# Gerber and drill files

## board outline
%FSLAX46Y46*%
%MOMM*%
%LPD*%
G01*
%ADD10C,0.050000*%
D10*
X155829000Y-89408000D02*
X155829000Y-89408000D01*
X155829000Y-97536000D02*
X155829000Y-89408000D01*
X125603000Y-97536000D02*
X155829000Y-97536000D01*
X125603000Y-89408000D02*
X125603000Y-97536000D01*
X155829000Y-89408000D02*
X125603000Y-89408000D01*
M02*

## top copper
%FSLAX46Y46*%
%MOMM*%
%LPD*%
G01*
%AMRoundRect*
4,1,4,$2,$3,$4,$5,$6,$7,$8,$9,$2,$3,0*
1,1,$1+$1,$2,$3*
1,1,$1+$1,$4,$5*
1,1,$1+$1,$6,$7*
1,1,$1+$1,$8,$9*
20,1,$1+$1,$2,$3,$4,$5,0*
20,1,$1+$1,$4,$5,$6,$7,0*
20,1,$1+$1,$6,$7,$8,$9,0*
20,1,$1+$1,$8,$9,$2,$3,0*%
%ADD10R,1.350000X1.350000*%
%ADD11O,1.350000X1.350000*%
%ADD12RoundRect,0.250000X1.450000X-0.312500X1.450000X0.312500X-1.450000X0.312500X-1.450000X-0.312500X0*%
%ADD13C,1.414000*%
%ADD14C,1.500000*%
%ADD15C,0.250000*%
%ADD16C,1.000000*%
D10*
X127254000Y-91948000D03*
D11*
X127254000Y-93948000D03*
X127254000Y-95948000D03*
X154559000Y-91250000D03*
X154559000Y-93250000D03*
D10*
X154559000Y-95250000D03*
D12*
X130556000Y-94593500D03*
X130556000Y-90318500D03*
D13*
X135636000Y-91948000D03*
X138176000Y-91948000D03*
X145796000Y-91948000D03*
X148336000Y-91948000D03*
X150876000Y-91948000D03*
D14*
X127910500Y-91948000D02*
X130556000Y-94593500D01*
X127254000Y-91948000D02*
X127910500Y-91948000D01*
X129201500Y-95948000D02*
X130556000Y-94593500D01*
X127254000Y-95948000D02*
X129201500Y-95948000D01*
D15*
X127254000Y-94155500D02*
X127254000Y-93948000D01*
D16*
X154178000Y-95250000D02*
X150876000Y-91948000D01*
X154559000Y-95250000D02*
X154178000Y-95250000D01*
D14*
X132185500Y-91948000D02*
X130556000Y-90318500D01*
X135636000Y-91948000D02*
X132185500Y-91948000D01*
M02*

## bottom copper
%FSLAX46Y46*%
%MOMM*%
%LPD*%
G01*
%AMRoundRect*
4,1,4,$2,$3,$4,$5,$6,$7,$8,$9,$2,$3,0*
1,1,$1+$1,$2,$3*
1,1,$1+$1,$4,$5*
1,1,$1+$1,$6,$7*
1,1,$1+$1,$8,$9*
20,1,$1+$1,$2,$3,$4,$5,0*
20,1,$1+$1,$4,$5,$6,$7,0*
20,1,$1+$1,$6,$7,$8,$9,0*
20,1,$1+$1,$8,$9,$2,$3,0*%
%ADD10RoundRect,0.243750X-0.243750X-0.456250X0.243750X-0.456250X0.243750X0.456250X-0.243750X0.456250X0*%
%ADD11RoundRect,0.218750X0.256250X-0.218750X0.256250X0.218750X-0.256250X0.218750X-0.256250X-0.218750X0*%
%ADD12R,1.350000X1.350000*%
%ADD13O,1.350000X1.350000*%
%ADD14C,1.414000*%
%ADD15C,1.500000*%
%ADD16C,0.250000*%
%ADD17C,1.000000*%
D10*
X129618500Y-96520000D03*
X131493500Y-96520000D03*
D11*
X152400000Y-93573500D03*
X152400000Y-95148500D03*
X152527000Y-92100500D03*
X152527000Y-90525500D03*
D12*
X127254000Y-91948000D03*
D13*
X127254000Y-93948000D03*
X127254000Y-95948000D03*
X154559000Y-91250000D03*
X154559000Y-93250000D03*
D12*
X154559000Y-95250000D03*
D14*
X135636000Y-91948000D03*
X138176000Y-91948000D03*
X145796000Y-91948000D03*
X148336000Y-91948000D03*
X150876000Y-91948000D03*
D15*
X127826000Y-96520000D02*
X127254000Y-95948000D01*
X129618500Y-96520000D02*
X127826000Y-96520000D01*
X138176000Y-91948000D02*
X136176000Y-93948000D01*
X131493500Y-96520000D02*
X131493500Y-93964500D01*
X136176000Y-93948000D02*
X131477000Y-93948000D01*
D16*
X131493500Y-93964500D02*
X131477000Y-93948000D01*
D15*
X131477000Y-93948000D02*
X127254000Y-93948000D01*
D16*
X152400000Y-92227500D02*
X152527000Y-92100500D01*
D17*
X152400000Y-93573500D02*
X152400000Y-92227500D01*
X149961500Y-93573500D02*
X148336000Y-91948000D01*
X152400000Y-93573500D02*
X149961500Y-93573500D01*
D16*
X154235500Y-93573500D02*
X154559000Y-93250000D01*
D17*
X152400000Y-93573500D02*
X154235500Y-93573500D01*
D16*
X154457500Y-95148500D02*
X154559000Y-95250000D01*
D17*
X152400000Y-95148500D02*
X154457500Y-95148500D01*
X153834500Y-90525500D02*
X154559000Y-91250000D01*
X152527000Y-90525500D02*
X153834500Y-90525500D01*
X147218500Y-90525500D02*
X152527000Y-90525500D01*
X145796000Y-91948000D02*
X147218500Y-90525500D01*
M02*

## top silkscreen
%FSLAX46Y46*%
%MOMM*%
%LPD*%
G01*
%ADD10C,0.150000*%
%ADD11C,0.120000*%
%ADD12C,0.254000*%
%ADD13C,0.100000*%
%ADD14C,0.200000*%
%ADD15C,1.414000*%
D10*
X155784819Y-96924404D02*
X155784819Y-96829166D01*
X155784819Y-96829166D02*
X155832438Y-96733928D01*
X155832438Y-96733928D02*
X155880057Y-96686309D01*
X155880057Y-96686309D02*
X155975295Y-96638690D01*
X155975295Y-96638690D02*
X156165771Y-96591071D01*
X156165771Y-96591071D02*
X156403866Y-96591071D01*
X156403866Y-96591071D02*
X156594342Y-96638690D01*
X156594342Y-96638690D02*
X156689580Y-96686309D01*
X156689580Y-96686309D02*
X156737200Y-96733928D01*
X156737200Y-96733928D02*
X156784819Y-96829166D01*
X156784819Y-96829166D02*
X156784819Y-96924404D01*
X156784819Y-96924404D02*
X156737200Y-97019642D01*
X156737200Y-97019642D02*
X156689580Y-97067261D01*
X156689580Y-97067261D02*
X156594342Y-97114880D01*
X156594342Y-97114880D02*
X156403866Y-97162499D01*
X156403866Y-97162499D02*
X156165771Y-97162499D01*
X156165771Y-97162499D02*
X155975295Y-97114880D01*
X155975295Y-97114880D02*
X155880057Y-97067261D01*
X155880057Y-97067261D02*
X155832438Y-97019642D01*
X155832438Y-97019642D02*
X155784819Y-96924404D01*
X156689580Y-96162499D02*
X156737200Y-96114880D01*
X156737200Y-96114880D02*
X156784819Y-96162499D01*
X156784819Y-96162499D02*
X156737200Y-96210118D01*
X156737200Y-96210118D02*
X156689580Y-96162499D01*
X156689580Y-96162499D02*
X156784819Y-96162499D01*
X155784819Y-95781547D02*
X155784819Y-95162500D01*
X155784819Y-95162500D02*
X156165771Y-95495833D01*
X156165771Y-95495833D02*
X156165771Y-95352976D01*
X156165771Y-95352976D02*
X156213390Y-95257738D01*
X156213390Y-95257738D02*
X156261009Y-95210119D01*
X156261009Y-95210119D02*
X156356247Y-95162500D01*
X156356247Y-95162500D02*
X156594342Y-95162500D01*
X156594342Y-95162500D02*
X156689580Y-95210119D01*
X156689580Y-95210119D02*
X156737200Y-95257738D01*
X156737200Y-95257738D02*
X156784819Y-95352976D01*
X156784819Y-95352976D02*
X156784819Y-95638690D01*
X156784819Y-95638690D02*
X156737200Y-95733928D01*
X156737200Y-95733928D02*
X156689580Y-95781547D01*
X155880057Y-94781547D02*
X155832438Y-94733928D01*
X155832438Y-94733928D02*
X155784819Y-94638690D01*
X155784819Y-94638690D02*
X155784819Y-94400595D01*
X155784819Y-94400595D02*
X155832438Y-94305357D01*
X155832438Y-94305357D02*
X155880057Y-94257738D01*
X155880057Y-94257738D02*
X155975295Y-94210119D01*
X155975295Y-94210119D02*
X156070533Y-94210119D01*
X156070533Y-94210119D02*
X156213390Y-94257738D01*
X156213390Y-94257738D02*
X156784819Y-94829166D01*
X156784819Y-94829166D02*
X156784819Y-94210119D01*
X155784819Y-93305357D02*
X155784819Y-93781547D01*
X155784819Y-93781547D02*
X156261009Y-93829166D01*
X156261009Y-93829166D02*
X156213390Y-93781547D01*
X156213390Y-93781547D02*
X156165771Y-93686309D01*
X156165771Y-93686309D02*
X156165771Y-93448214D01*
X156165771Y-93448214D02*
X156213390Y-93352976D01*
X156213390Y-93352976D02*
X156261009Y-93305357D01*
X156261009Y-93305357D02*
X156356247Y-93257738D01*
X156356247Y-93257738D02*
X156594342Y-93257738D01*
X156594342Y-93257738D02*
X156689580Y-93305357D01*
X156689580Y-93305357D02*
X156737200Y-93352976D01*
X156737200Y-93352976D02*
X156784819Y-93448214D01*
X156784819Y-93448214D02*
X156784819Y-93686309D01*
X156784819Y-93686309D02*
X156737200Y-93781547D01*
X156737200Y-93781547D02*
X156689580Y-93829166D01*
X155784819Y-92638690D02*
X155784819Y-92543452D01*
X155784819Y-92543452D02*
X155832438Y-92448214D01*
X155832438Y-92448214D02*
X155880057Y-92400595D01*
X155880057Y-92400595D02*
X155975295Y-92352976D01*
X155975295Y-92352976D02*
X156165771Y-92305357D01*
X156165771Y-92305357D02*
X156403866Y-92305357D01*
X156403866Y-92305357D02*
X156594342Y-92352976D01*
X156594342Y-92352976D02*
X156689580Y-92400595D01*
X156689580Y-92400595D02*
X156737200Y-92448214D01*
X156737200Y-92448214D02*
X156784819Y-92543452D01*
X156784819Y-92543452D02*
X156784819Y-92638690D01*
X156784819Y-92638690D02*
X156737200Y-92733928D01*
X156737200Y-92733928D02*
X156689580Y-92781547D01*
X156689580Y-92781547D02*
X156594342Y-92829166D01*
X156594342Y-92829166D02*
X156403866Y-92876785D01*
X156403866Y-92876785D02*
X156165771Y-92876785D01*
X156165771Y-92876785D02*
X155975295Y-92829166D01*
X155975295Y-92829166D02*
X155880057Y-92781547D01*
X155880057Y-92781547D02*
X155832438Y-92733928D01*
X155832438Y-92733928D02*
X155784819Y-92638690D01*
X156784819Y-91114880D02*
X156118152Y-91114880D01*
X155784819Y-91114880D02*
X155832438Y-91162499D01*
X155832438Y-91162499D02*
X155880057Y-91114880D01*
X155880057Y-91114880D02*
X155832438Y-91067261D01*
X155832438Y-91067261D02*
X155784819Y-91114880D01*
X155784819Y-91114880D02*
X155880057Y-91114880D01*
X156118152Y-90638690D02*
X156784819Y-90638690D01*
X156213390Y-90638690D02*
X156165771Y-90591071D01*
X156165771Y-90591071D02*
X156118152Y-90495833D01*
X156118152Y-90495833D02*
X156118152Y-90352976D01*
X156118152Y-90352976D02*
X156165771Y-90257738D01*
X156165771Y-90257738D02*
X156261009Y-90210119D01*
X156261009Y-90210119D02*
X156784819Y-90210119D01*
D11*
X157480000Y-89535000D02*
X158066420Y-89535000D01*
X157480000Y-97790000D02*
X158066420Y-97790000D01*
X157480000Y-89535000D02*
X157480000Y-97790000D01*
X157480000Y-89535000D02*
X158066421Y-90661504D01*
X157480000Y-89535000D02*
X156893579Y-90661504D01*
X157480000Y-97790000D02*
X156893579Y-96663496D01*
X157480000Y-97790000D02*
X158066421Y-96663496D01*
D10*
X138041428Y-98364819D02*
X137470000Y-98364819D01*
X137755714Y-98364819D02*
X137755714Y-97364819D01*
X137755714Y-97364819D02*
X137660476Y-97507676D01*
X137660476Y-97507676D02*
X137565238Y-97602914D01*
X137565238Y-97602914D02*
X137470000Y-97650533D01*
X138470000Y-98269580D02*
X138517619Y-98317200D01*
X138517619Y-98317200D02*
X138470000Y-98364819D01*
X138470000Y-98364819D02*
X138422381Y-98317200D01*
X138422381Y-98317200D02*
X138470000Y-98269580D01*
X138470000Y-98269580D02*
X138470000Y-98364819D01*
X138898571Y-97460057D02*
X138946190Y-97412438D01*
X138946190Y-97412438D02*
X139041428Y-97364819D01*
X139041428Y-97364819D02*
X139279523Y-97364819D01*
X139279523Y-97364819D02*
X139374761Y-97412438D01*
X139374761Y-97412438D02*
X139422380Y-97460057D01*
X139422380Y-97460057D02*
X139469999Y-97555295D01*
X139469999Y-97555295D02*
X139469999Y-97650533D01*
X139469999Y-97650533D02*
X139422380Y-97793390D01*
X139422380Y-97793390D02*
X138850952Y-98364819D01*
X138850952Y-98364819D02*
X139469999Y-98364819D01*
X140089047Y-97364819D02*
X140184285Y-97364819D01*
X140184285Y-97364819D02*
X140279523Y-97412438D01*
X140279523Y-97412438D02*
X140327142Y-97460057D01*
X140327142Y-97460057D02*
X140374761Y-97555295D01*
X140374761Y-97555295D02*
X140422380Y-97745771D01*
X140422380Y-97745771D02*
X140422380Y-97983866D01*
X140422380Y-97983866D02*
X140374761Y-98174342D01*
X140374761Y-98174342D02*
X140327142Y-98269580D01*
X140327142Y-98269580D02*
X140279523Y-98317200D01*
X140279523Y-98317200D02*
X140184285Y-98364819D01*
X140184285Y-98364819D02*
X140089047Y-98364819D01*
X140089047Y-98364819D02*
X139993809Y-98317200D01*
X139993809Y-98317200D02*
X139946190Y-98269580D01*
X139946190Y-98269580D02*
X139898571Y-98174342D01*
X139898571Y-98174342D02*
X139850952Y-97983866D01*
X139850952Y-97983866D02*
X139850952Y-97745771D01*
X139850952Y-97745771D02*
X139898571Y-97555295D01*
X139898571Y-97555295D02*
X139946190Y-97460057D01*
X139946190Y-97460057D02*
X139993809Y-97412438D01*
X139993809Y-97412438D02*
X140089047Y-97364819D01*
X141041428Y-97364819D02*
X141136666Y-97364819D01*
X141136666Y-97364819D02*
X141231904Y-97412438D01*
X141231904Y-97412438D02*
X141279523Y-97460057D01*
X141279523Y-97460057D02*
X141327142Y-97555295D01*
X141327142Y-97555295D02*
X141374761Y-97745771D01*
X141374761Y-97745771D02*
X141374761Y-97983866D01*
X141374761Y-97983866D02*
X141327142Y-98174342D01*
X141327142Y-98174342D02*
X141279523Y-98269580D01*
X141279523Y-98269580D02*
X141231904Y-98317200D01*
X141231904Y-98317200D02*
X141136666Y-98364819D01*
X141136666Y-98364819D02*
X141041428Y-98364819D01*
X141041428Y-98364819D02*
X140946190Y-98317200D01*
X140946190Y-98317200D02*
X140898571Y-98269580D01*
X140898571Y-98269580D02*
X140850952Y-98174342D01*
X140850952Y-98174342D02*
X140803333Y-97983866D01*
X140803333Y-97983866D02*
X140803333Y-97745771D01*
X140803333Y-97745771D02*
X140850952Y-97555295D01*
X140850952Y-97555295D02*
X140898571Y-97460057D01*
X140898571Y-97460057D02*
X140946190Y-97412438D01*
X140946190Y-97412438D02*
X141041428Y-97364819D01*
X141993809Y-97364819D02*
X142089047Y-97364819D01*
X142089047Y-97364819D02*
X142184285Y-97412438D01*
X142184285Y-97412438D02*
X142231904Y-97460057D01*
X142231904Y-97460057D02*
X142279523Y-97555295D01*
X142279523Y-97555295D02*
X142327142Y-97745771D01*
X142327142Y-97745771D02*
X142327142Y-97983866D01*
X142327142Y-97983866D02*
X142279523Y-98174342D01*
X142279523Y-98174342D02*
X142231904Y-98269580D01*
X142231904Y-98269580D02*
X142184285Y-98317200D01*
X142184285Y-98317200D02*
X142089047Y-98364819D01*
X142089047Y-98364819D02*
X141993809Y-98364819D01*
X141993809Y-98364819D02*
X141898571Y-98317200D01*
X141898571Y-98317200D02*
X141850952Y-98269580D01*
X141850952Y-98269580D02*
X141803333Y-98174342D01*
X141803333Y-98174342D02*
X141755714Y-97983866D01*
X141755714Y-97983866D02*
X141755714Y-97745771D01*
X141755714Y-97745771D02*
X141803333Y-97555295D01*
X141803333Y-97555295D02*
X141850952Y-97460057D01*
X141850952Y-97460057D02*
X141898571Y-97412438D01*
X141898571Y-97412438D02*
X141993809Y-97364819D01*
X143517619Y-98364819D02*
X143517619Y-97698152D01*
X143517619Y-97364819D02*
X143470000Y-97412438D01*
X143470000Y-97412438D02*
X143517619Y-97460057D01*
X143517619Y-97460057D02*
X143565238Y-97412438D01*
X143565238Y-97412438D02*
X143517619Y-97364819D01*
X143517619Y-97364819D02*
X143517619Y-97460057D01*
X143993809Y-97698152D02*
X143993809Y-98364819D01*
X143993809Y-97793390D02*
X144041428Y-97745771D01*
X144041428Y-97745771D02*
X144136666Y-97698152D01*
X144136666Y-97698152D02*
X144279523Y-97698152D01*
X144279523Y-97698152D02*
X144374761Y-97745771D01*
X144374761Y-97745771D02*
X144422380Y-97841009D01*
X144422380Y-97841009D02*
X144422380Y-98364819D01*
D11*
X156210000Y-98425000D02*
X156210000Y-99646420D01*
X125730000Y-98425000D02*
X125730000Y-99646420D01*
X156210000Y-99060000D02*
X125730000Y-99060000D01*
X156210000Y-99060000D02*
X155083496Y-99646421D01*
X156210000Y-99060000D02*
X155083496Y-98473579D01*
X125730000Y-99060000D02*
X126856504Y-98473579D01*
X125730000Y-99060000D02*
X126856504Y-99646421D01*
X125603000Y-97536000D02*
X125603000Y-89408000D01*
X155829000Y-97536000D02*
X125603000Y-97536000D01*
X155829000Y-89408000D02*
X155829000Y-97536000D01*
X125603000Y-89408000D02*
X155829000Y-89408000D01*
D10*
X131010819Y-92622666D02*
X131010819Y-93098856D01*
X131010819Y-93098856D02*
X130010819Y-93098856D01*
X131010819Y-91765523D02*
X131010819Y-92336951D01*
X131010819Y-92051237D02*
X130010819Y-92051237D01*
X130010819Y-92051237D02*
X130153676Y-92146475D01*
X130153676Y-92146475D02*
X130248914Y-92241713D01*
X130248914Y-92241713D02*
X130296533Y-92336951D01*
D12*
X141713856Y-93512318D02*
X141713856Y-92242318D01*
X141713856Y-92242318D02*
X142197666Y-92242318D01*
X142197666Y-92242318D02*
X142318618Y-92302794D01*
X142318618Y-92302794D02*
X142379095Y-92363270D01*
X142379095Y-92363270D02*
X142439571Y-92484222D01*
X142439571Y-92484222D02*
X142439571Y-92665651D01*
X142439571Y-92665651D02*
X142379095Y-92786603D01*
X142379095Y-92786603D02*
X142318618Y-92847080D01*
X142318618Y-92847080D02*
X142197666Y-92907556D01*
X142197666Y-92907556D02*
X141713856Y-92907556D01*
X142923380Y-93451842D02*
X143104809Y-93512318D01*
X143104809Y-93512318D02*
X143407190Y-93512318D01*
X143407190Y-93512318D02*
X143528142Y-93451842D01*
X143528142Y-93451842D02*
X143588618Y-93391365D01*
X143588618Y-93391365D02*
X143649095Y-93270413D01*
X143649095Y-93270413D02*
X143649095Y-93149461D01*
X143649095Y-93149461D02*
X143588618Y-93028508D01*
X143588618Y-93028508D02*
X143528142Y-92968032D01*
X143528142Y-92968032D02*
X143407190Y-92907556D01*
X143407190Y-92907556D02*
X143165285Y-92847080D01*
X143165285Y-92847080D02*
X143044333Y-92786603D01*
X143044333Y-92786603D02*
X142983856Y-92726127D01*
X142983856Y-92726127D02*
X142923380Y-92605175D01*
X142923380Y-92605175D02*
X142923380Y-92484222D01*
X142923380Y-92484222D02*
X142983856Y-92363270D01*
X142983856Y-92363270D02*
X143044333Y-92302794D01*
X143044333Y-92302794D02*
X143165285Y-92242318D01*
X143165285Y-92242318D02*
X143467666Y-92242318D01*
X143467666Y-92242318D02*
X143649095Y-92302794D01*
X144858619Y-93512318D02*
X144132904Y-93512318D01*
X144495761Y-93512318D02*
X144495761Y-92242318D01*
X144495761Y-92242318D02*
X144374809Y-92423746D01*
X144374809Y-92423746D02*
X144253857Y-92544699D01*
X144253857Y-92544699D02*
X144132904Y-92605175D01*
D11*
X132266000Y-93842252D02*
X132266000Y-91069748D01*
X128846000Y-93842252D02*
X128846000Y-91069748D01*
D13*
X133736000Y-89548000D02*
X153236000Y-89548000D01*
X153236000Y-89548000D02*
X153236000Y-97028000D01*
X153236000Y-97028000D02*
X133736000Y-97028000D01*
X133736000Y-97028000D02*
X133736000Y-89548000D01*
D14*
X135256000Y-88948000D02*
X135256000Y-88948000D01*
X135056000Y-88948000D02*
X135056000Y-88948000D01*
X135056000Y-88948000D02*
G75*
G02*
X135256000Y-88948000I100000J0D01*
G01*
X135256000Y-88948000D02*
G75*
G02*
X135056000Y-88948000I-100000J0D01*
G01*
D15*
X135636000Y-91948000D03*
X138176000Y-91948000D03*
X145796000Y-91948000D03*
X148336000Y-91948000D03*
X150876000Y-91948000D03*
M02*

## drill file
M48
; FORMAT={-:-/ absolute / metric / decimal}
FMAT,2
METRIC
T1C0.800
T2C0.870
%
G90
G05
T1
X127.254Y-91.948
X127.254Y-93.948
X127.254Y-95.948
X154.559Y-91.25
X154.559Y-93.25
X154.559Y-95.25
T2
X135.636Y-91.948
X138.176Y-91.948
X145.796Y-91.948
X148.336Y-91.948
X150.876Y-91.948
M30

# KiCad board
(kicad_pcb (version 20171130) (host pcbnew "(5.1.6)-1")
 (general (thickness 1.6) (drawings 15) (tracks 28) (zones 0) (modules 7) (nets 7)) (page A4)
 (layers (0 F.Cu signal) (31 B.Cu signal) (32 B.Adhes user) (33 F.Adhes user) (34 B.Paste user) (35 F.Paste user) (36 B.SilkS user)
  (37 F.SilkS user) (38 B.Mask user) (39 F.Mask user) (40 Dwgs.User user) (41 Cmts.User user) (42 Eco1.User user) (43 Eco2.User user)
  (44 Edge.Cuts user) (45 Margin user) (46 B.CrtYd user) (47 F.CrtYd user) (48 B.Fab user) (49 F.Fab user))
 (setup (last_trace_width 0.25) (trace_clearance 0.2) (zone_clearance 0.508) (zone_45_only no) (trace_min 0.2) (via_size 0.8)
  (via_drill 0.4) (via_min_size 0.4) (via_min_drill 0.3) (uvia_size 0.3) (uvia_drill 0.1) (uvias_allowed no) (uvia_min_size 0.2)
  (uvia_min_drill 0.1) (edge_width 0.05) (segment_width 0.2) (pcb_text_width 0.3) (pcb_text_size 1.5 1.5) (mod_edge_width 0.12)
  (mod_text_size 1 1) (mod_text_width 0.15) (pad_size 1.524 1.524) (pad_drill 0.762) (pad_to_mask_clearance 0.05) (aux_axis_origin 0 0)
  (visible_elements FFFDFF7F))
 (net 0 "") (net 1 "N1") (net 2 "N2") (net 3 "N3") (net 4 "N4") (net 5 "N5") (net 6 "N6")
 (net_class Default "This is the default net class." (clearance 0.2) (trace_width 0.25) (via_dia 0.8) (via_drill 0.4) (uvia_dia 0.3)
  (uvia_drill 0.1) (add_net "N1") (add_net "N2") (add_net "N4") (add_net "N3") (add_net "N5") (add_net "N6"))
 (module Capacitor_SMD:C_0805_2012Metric (layer B.Cu) (at 130.556 96.52)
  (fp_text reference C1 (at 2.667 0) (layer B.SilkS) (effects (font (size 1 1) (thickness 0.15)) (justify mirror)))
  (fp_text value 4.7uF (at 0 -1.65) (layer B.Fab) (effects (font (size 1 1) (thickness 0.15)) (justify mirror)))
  (pad 1 smd roundrect (at -0.9375 0) (size 0.975 1.4) (layers B.Cu B.Paste B.Mask) (roundrect_rratio 0.25) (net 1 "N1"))
  (pad 2 smd roundrect (at 0.9375 0) (size 0.975 1.4) (layers B.Cu B.Paste B.Mask) (roundrect_rratio 0.25) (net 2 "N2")))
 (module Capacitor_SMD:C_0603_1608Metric (layer B.Cu) (at 152.4 94.361 90)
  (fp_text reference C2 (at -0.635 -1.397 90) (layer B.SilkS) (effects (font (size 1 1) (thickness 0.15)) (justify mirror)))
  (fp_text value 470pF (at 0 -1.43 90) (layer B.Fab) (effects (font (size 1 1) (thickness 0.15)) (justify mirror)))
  (pad 2 smd roundrect (at 0.7875 0 90) (size 0.875 0.95) (layers B.Cu B.Paste B.Mask) (roundrect_rratio 0.25) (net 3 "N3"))
  (pad 1 smd roundrect (at -0.7875 0 90) (size 0.875 0.95) (layers B.Cu B.Paste B.Mask) (roundrect_rratio 0.25) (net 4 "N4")))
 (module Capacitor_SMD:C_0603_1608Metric (layer B.Cu) (at 152.527 91.313 90)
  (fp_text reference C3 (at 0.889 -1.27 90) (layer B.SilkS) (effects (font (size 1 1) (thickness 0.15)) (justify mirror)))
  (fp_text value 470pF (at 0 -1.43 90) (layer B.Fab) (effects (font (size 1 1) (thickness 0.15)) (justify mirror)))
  (pad 1 smd roundrect (at -0.7875 0 90) (size 0.875 0.95) (layers B.Cu B.Paste B.Mask) (roundrect_rratio 0.25) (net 3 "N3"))
  (pad 2 smd roundrect (at 0.7875 0 90) (size 0.875 0.95) (layers B.Cu B.Paste B.Mask) (roundrect_rratio 0.25) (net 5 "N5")))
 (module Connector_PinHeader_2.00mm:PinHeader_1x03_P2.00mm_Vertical (layer B.Cu) (at 127.254 91.948 180)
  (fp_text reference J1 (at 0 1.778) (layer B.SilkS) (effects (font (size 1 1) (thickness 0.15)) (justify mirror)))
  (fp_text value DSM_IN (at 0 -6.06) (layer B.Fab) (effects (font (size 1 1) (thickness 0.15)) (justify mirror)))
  (pad 1 thru_hole rect (at 0 0 180) (size 1.35 1.35) (drill 0.8) (layers *.Cu *.Mask) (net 1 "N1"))
  (pad 2 thru_hole oval (at 0 -2 180) (size 1.35 1.35) (drill 0.8) (layers *.Cu *.Mask) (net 2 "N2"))
  (pad 3 thru_hole oval (at 0 -4 180) (size 1.35 1.35) (drill 0.8) (layers *.Cu *.Mask) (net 1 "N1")))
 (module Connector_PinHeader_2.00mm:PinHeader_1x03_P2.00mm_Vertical (layer B.Cu) (at 154.559 95.25)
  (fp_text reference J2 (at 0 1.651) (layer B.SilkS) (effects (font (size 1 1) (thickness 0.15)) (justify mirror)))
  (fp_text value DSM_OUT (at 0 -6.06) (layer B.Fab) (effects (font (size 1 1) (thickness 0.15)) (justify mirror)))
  (pad 3 thru_hole oval (at 0 -4) (size 1.35 1.35) (drill 0.8) (layers *.Cu *.Mask) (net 5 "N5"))
  (pad 2 thru_hole oval (at 0 -2) (size 1.35 1.35) (drill 0.8) (layers *.Cu *.Mask) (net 3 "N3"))
  (pad 1 thru_hole rect (at 0 0) (size 1.35 1.35) (drill 0.8) (layers *.Cu *.Mask) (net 4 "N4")))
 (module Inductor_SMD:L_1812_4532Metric (layer F.Cu) (at 130.556 92.456 90)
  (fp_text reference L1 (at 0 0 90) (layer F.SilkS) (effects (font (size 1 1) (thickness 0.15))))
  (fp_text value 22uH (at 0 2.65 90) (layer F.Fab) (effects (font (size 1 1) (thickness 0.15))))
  (fp_line (start -1.386252 1.71) (end 1.386252 1.71) (layer F.SilkS) (width 0.12))
  (fp_line (start -1.386252 -1.71) (end 1.386252 -1.71) (layer F.SilkS) (width 0.12))
  (pad 1 smd roundrect (at -2.1375 0 90) (size 1.125 3.4) (layers F.Cu F.Paste F.Mask) (roundrect_rratio 0.222222) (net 1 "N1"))
  (pad 2 smd roundrect (at 2.1375 0 90) (size 1.125 3.4) (layers F.Cu F.Paste F.Mask) (roundrect_rratio 0.222222) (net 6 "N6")))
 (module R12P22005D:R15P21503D (layer F.Cu) (at 135.636 91.948)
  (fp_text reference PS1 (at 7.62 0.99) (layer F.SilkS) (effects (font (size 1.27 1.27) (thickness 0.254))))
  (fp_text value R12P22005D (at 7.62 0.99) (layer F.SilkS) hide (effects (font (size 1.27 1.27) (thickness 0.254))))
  (fp_line (start -1.9 -2.4) (end 17.6 -2.4) (layer F.SilkS) (width 0.1))
  (fp_line (start 17.6 -2.4) (end 17.6 5.08) (layer F.SilkS) (width 0.1))
  (fp_line (start 17.6 5.08) (end -1.9 5.08) (layer F.SilkS) (width 0.1))
  (fp_line (start -1.9 5.08) (end -1.9 -2.4) (layer F.SilkS) (width 0.1))
  (fp_line (start -0.38 -3) (end -0.38 -3) (layer F.SilkS) (width 0.2))
  (fp_line (start -0.58 -3) (end -0.58 -3) (layer F.SilkS) (width 0.2))
  (fp_arc (start -0.48 -3) (end -0.38 -3) (angle -180) (layer F.SilkS) (width 0.2))
  (fp_arc (start -0.48 -3) (end -0.58 -3) (angle -180) (layer F.SilkS) (width 0.2))
  (pad 1 thru_hole circle (at 0 0 90) (size 1.414 1.414) (drill 0.87) (layers *.Cu *.Mask F.SilkS) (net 6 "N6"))
  (pad 2 thru_hole circle (at 2.54 0 90) (size 1.414 1.414) (drill 0.87) (layers *.Cu *.Mask F.SilkS) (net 2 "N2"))
  (pad 5 thru_hole circle (at 10.16 0 90) (size 1.414 1.414) (drill 0.87) (layers *.Cu *.Mask F.SilkS) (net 5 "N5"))
  (pad 6 thru_hole circle (at 12.7 0 90) (size 1.414 1.414) (drill 0.87) (layers *.Cu *.Mask F.SilkS) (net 3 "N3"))
  (pad 7 thru_hole circle (at 15.24 0 90) (size 1.414 1.414) (drill 0.87) (layers *.Cu *.Mask F.SilkS) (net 4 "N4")))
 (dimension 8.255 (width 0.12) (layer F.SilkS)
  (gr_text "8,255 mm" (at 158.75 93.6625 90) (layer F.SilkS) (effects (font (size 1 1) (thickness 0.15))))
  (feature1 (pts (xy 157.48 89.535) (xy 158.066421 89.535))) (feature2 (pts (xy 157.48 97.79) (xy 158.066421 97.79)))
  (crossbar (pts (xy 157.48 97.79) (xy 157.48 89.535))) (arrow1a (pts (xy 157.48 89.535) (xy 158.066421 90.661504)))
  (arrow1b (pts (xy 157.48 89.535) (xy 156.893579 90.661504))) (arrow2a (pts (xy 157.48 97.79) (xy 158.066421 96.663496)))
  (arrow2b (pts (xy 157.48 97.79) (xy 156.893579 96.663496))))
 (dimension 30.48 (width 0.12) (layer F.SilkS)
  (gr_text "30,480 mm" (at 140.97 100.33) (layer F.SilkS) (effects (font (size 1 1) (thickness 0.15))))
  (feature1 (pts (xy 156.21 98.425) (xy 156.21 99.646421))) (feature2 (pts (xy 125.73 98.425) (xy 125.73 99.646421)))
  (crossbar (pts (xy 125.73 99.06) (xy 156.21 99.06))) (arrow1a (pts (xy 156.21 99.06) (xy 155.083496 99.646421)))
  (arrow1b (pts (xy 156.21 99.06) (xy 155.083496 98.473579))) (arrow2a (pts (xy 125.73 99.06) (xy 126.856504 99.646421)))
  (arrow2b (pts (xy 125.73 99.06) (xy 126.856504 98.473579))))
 (gr_line (start 125.603 97.536) (end 125.603 89.408) (layer F.SilkS) (width 0.12))
 (gr_line (start 155.829 97.536) (end 125.603 97.536) (layer F.SilkS) (width 0.12))
 (gr_line (start 155.829 89.408) (end 155.829 97.536) (layer F.SilkS) (width 0.12))
 (gr_line (start 125.603 89.408) (end 155.829 89.408) (layer F.SilkS) (width 0.12))
 (gr_line (start 155.829 89.408) (end 155.829 89.408) (layer Edge.Cuts) (width 0.05))
 (gr_line (start 155.829 97.536) (end 155.829 89.408) (layer Edge.Cuts) (width 0.05))
 (gr_line (start 125.603 97.536) (end 155.829 97.536) (layer Edge.Cuts) (width 0.05))
 (gr_line (start 125.603 89.408) (end 125.603 97.536) (layer Edge.Cuts) (width 0.05))
 (gr_line (start 155.829 89.408) (end 125.603 89.408) (layer Edge.Cuts) (width 0.05))
 (segment (start 127.9105 91.948) (end 130.556 94.5935) (width 1.5) (layer F.Cu) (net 1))
 (segment (start 127.254 91.948) (end 127.9105 91.948) (width 1.5) (layer F.Cu) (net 1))
 (segment (start 127.826 96.52) (end 127.254 95.948) (width 1.5) (layer B.Cu) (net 1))
 (segment (start 129.6185 96.52) (end 127.826 96.52) (width 1.5) (layer B.Cu) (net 1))
 (segment (start 129.2015 95.948) (end 130.556 94.5935) (width 1.5) (layer F.Cu) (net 1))
 (segment (start 127.254 95.948) (end 129.2015 95.948) (width 1.5) (layer F.Cu) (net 1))
 (segment (start 127.254 94.1555) (end 127.254 93.948) (width 0.25) (layer F.Cu) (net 2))
 (segment (start 138.176 91.948) (end 136.176 93.948) (width 1.5) (layer B.Cu) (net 2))
 (segment (start 131.4935 96.52) (end 131.4935 93.9645) (width 1.5) (layer B.Cu) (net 2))
 (segment (start 136.176 93.948) (end 131.477 93.948) (width 1.5) (layer B.Cu) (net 2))
 (segment (start 131.4935 93.9645) (end 131.477 93.948) (width 0.25) (layer B.Cu) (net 2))
 (segment (start 131.477 93.948) (end 127.254 93.948) (width 1.5) (layer B.Cu) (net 2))
 (segment (start 152.4 92.2275) (end 152.527 92.1005) (width 0.25) (layer B.Cu) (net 3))
 (segment (start 152.4 93.5735) (end 152.4 92.2275) (width 1) (layer B.Cu) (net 3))
 (segment (start 149.9615 93.5735) (end 148.336 91.948) (width 1) (layer B.Cu) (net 3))
 (segment (start 152.4 93.5735) (end 149.9615 93.5735) (width 1) (layer B.Cu) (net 3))
 (segment (start 154.2355 93.5735) (end 154.559 93.25) (width 0.25) (layer B.Cu) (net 3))
 (segment (start 152.4 93.5735) (end 154.2355 93.5735) (width 1) (layer B.Cu) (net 3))
 (segment (start 154.4575 95.1485) (end 154.559 95.25) (width 0.25) (layer B.Cu) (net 4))
 (segment (start 152.4 95.1485) (end 154.4575 95.1485) (width 1) (layer B.Cu) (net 4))
 (segment (start 154.178 95.25) (end 150.876 91.948) (width 1) (layer F.Cu) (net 4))
 (segment (start 154.559 95.25) (end 154.178 95.25) (width 1) (layer F.Cu) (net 4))
 (segment (start 153.8345 90.5255) (end 154.559 91.25) (width 1) (layer B.Cu) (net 5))
 (segment (start 152.527 90.5255) (end 153.8345 90.5255) (width 1) (layer B.Cu) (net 5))
 (segment (start 147.2185 90.5255) (end 152.527 90.5255) (width 1) (layer B.Cu) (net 5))
 (segment (start 145.796 91.948) (end 147.2185 90.5255) (width 1) (layer B.Cu) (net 5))
 (segment (start 132.1855 91.948) (end 130.556 90.3185) (width 1.5) (layer F.Cu) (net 6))
 (segment (start 135.636 91.948) (end 132.1855 91.948) (width 1.5) (layer F.Cu) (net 6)))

